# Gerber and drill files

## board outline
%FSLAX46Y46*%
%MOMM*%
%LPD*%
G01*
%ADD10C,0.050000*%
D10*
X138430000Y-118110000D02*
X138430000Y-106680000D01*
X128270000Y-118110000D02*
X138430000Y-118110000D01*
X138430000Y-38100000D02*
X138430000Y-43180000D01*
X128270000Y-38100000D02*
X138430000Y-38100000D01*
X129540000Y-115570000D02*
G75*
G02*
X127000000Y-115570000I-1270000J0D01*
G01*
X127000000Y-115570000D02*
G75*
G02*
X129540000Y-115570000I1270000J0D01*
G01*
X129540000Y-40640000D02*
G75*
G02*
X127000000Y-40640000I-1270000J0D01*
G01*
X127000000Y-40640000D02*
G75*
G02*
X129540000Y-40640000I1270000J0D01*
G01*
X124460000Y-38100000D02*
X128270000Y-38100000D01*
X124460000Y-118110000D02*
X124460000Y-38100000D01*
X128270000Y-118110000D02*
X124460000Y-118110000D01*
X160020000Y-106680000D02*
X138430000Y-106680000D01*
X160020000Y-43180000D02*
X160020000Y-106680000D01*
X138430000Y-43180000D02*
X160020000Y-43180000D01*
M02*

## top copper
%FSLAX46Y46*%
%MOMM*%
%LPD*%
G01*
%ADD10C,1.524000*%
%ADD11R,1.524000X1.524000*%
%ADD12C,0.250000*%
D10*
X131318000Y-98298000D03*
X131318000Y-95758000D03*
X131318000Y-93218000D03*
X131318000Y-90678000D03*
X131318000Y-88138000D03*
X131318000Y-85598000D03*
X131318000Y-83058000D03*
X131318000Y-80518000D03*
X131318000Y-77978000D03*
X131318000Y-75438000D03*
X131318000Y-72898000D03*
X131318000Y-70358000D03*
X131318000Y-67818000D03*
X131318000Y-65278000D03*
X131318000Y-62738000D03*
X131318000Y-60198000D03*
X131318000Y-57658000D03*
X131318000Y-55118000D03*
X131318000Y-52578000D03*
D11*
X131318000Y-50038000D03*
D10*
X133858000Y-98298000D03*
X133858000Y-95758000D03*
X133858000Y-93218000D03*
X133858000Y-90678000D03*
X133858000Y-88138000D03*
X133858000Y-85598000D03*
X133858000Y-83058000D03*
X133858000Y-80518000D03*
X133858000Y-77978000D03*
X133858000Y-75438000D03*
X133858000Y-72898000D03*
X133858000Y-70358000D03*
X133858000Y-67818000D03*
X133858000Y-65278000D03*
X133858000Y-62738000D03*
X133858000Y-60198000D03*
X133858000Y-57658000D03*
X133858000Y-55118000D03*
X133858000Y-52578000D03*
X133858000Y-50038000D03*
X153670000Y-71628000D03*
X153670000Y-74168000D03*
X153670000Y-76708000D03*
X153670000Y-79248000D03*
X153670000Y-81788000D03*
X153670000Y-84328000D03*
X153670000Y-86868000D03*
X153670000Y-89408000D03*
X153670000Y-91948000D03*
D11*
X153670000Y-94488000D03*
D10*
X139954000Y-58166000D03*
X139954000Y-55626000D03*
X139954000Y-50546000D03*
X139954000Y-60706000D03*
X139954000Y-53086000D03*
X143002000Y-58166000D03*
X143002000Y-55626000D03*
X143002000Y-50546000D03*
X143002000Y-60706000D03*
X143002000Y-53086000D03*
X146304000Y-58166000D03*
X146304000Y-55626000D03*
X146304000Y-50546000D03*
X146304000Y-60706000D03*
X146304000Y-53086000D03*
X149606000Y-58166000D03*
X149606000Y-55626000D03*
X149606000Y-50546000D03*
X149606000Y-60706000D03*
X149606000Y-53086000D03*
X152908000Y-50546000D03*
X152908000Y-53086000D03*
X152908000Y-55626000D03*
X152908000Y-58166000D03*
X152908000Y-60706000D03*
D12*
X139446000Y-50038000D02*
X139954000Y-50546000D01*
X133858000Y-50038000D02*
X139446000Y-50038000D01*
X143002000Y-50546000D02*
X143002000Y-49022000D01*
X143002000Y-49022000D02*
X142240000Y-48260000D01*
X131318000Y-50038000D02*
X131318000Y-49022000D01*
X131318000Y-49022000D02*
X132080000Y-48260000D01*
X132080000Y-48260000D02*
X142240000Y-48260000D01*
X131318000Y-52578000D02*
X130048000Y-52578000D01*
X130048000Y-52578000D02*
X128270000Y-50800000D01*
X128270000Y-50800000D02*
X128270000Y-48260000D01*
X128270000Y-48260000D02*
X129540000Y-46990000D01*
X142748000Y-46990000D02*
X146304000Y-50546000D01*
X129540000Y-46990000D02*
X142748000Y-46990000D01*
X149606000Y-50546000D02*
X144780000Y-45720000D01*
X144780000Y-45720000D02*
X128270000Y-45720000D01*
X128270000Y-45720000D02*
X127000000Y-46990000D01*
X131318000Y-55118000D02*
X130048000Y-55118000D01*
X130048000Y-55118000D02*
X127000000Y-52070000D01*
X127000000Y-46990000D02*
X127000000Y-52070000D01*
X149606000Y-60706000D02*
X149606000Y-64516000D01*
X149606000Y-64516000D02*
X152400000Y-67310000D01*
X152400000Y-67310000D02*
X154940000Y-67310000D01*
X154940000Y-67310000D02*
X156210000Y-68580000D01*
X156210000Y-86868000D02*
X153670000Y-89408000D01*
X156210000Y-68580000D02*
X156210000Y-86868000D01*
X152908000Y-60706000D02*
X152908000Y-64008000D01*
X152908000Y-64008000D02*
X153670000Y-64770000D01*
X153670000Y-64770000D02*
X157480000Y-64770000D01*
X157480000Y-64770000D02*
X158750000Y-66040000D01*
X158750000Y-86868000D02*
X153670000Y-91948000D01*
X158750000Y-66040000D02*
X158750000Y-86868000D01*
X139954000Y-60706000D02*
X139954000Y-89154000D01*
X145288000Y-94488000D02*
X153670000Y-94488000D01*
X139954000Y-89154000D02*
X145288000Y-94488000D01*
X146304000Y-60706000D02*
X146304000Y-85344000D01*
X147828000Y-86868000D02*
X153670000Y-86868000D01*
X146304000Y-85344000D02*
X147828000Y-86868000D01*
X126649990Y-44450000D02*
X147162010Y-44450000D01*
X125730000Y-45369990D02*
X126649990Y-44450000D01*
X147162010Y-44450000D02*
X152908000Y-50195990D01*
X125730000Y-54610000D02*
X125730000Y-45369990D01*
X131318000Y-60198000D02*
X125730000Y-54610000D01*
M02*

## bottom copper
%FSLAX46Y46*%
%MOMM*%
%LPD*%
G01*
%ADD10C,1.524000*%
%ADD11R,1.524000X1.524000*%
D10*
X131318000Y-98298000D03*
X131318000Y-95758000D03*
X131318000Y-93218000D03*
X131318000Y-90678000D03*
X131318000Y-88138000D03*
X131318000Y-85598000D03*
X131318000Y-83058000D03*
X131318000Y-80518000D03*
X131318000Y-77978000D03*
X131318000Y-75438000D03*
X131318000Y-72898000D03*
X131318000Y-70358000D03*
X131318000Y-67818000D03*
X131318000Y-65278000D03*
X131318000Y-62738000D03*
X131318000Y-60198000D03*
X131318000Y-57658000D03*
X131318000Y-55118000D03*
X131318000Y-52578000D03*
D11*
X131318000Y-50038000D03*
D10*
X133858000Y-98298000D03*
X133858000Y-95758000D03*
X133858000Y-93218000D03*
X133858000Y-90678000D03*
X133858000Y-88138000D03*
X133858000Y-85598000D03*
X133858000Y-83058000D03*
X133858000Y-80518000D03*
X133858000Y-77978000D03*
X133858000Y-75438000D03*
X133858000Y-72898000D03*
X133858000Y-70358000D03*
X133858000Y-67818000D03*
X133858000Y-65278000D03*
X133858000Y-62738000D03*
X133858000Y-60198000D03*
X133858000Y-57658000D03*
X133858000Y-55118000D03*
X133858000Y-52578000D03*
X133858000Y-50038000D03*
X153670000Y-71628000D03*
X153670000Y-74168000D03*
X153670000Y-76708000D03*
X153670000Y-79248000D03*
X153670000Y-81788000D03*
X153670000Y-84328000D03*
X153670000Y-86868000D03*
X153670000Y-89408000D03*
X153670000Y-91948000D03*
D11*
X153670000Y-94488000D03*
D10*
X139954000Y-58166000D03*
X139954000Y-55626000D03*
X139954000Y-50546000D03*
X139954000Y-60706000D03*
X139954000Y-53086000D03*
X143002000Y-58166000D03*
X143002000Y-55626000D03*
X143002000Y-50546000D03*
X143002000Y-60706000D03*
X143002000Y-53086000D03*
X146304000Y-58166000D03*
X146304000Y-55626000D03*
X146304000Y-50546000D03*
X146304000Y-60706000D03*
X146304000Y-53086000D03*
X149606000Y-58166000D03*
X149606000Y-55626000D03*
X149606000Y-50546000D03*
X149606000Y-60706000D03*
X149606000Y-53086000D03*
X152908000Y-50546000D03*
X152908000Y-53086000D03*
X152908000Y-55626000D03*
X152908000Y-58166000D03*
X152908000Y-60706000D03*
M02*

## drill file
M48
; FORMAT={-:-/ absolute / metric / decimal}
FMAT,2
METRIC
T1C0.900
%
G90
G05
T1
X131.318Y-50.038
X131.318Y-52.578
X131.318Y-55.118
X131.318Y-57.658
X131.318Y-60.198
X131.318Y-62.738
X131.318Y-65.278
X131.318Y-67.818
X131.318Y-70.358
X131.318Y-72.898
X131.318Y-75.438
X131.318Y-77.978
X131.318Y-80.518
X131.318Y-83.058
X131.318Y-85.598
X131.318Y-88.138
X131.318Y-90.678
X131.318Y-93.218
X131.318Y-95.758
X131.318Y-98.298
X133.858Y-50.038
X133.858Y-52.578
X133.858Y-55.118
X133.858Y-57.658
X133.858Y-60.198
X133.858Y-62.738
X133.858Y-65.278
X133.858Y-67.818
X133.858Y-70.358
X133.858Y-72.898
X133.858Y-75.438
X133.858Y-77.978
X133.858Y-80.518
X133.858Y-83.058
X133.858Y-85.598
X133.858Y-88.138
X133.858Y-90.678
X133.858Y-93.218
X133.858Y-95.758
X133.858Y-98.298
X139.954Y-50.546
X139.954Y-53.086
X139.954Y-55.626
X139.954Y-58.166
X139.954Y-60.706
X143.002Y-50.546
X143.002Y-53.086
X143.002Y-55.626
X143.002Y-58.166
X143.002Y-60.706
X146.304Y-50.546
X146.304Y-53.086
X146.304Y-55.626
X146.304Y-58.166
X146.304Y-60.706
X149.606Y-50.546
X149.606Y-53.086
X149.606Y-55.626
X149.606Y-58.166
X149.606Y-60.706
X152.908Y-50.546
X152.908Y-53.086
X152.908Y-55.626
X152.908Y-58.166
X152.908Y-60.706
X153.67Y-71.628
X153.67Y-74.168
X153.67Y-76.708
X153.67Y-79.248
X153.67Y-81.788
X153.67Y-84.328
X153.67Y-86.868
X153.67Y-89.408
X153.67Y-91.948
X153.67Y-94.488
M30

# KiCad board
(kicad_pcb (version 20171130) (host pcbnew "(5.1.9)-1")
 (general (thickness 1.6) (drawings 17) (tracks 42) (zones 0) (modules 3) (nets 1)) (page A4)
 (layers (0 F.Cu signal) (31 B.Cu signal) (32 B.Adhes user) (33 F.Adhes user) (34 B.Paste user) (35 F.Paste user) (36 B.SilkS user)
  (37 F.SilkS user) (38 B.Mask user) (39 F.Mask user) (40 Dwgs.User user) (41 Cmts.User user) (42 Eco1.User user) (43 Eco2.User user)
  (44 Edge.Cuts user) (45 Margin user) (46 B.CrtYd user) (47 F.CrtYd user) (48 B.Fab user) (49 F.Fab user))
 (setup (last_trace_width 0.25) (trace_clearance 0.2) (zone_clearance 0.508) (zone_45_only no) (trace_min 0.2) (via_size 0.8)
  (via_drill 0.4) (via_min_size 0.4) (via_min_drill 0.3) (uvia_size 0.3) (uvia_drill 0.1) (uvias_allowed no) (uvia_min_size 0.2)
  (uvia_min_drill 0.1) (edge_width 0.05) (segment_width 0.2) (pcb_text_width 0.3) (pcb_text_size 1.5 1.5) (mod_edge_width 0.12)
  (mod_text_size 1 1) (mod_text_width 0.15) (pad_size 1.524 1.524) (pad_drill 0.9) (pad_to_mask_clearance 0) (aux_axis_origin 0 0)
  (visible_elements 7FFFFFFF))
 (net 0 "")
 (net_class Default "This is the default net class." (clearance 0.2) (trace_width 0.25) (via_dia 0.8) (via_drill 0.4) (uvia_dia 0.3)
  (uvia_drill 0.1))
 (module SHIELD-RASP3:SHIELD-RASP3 (layer F.Cu) (at 118.11 100.33)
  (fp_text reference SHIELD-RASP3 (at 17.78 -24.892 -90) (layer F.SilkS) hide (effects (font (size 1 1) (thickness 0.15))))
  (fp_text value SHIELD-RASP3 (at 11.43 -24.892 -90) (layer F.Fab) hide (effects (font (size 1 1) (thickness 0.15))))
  (pad 39 thru_hole circle (at 13.208 -2.032 270) (size 1.524 1.524) (drill 0.9) (layers *.Cu *.Mask))
  (pad 37 thru_hole circle (at 13.208 -4.572 270) (size 1.524 1.524) (drill 0.9) (layers *.Cu *.Mask))
  (pad 35 thru_hole circle (at 13.208 -7.112 270) (size 1.524 1.524) (drill 0.9) (layers *.Cu *.Mask))
  (pad 33 thru_hole circle (at 13.208 -9.652 270) (size 1.524 1.524) (drill 0.9) (layers *.Cu *.Mask))
  (pad 31 thru_hole circle (at 13.208 -12.192 270) (size 1.524 1.524) (drill 0.9) (layers *.Cu *.Mask))
  (pad 29 thru_hole circle (at 13.208 -14.732 270) (size 1.524 1.524) (drill 0.9) (layers *.Cu *.Mask))
  (pad 27 thru_hole circle (at 13.208 -17.272 270) (size 1.524 1.524) (drill 0.9) (layers *.Cu *.Mask))
  (pad 25 thru_hole circle (at 13.208 -19.812 270) (size 1.524 1.524) (drill 0.9) (layers *.Cu *.Mask))
  (pad 23 thru_hole circle (at 13.208 -22.352 270) (size 1.524 1.524) (drill 0.9) (layers *.Cu *.Mask))
  (pad 21 thru_hole circle (at 13.208 -24.892 270) (size 1.524 1.524) (drill 0.9) (layers *.Cu *.Mask))
  (pad 19 thru_hole circle (at 13.208 -27.432 270) (size 1.524 1.524) (drill 0.9) (layers *.Cu *.Mask))
  (pad 17 thru_hole circle (at 13.208 -29.972 270) (size 1.524 1.524) (drill 0.9) (layers *.Cu *.Mask))
  (pad 15 thru_hole circle (at 13.208 -32.512 270) (size 1.524 1.524) (drill 0.9) (layers *.Cu *.Mask))
  (pad 13 thru_hole circle (at 13.208 -35.052 270) (size 1.524 1.524) (drill 0.9) (layers *.Cu *.Mask))
  (pad 11 thru_hole circle (at 13.208 -37.592 270) (size 1.524 1.524) (drill 0.9) (layers *.Cu *.Mask))
  (pad 9 thru_hole circle (at 13.208 -40.132 270) (size 1.524 1.524) (drill 0.9) (layers *.Cu *.Mask))
  (pad 7 thru_hole circle (at 13.208 -42.672 270) (size 1.524 1.524) (drill 0.9) (layers *.Cu *.Mask F.Paste))
  (pad 5 thru_hole circle (at 13.208 -45.212 270) (size 1.524 1.524) (drill 0.9) (layers *.Cu *.Mask))
  (pad 3 thru_hole circle (at 13.208 -47.752 270) (size 1.524 1.524) (drill 0.9) (layers *.Cu *.Mask))
  (pad 1 thru_hole rect (at 13.208 -50.292 270) (size 1.524 1.524) (drill 0.9) (layers *.Cu *.Mask))
  (pad 40 thru_hole circle (at 15.748 -2.032 270) (size 1.524 1.524) (drill 0.9) (layers *.Cu *.Mask))
  (pad 38 thru_hole circle (at 15.748 -4.572 270) (size 1.524 1.524) (drill 0.9) (layers *.Cu *.Mask))
  (pad 36 thru_hole circle (at 15.748 -7.112 270) (size 1.524 1.524) (drill 0.9) (layers *.Cu *.Mask))
  (pad 34 thru_hole circle (at 15.748 -9.652 270) (size 1.524 1.524) (drill 0.9) (layers *.Cu *.Mask))
  (pad 32 thru_hole circle (at 15.748 -12.192 270) (size 1.524 1.524) (drill 0.9) (layers *.Cu *.Mask))
  (pad 30 thru_hole circle (at 15.748 -14.732 270) (size 1.524 1.524) (drill 0.9) (layers *.Cu *.Mask))
  (pad 28 thru_hole circle (at 15.748 -17.272 270) (size 1.524 1.524) (drill 0.9) (layers *.Cu *.Mask))
  (pad 26 thru_hole circle (at 15.748 -19.812 270) (size 1.524 1.524) (drill 0.9) (layers *.Cu *.Mask))
  (pad 24 thru_hole circle (at 15.748 -22.352 270) (size 1.524 1.524) (drill 0.9) (layers *.Cu *.Mask))
  (pad 22 thru_hole circle (at 15.748 -24.892 270) (size 1.524 1.524) (drill 0.9) (layers *.Cu *.Mask))
  (pad 20 thru_hole circle (at 15.748 -27.432 270) (size 1.524 1.524) (drill 0.9) (layers *.Cu *.Mask))
  (pad 18 thru_hole circle (at 15.748 -29.972 270) (size 1.524 1.524) (drill 0.9) (layers *.Cu *.Mask))
  (pad 16 thru_hole circle (at 15.748 -32.512 270) (size 1.524 1.524) (drill 0.9) (layers *.Cu *.Mask))
  (pad 14 thru_hole circle (at 15.748 -35.052 270) (size 1.524 1.524) (drill 0.9) (layers *.Cu *.Mask))
  (pad 12 thru_hole circle (at 15.748 -37.592 270) (size 1.524 1.524) (drill 0.9) (layers *.Cu *.Mask))
  (pad 10 thru_hole circle (at 15.748 -40.132 270) (size 1.524 1.524) (drill 0.9) (layers *.Cu *.Mask))
  (pad 8 thru_hole circle (at 15.748 -42.672 270) (size 1.524 1.524) (drill 0.9) (layers *.Cu *.Mask))
  (pad 6 thru_hole circle (at 15.748 -45.212 270) (size 1.524 1.524) (drill 0.9) (layers *.Cu *.Mask))
  (pad 4 thru_hole circle (at 15.748 -47.752 270) (size 1.524 1.524) (drill 0.9) (layers *.Cu *.Mask))
  (pad 2 thru_hole circle (at 15.748 -50.292 270) (size 1.524 1.524) (drill 0.9) (layers *.Cu *.Mask)))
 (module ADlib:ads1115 (layer F.Cu) (at 148.59 92.71 90)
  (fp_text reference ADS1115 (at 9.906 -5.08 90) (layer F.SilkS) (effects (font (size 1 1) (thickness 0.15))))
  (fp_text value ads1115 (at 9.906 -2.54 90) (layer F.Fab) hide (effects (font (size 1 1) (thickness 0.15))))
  (pad 10 thru_hole circle (at 21.082 5.08 90) (size 1.524 1.524) (drill 0.9) (layers *.Cu *.Mask))
  (pad 9 thru_hole circle (at 18.542 5.08 90) (size 1.524 1.524) (drill 0.9) (layers *.Cu *.Mask))
  (pad 8 thru_hole circle (at 16.002 5.08 90) (size 1.524 1.524) (drill 0.9) (layers *.Cu *.Mask))
  (pad 7 thru_hole circle (at 13.462 5.08 90) (size 1.524 1.524) (drill 0.9) (layers *.Cu *.Mask))
  (pad 6 thru_hole circle (at 10.922 5.08 90) (size 1.524 1.524) (drill 0.9) (layers *.Cu *.Mask))
  (pad 5 thru_hole circle (at 8.382 5.08 90) (size 1.524 1.524) (drill 0.9) (layers *.Cu *.Mask))
  (pad 4 thru_hole circle (at 5.842 5.08 90) (size 1.524 1.524) (drill 0.9) (layers *.Cu *.Mask))
  (pad 3 thru_hole circle (at 3.302 5.08 90) (size 1.524 1.524) (drill 0.9) (layers *.Cu *.Mask))
  (pad 2 thru_hole circle (at 0.762 5.08 90) (size 1.524 1.524) (drill 0.9) (layers *.Cu *.Mask))
  (pad 1 thru_hole rect (at -1.778 5.08 90) (size 1.524 1.524) (drill 0.9) (layers *.Cu *.Mask)))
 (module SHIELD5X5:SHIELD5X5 (layer F.Cu) (at 154.94 54.61 180)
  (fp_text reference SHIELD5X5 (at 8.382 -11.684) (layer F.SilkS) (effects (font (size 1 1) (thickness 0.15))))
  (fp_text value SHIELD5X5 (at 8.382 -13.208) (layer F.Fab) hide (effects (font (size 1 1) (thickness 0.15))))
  (pad 2 thru_hole circle (at 14.986 -3.556 180) (size 1.524 1.524) (drill 0.9) (layers *.Cu *.Mask))
  (pad 3 thru_hole circle (at 14.986 -1.016 180) (size 1.524 1.524) (drill 0.9) (layers *.Cu *.Mask))
  (pad 5 thru_hole circle (at 14.986 4.064 180) (size 1.524 1.524) (drill 0.9) (layers *.Cu *.Mask))
  (pad 1 thru_hole circle (at 14.986 -6.096 180) (size 1.524 1.524) (drill 0.9) (layers *.Cu *.Mask))
  (pad 4 thru_hole circle (at 14.986 1.524 180) (size 1.524 1.524) (drill 0.9) (layers *.Cu *.Mask))
  (pad 2 thru_hole circle (at 11.938 -3.556 180) (size 1.524 1.524) (drill 0.9) (layers *.Cu *.Mask))
  (pad 3 thru_hole circle (at 11.938 -1.016 180) (size 1.524 1.524) (drill 0.9) (layers *.Cu *.Mask))
  (pad 5 thru_hole circle (at 11.938 4.064 180) (size 1.524 1.524) (drill 0.9) (layers *.Cu *.Mask))
  (pad 1 thru_hole circle (at 11.938 -6.096 180) (size 1.524 1.524) (drill 0.9) (layers *.Cu *.Mask))
  (pad 4 thru_hole circle (at 11.938 1.524 180) (size 1.524 1.524) (drill 0.9) (layers *.Cu *.Mask))
  (pad 2 thru_hole circle (at 8.636 -3.556 180) (size 1.524 1.524) (drill 0.9) (layers *.Cu *.Mask))
  (pad 3 thru_hole circle (at 8.636 -1.016 180) (size 1.524 1.524) (drill 0.9) (layers *.Cu *.Mask))
  (pad 5 thru_hole circle (at 8.636 4.064 180) (size 1.524 1.524) (drill 0.9) (layers *.Cu *.Mask))
  (pad 1 thru_hole circle (at 8.636 -6.096 180) (size 1.524 1.524) (drill 0.9) (layers *.Cu *.Mask))
  (pad 4 thru_hole circle (at 8.636 1.524 180) (size 1.524 1.524) (drill 0.9) (layers *.Cu *.Mask))
  (pad 2 thru_hole circle (at 5.334 -3.556 180) (size 1.524 1.524) (drill 0.9) (layers *.Cu *.Mask))
  (pad 3 thru_hole circle (at 5.334 -1.016 180) (size 1.524 1.524) (drill 0.9) (layers *.Cu *.Mask))
  (pad 5 thru_hole circle (at 5.334 4.064 180) (size 1.524 1.524) (drill 0.9) (layers *.Cu *.Mask))
  (pad 1 thru_hole circle (at 5.334 -6.096 180) (size 1.524 1.524) (drill 0.9) (layers *.Cu *.Mask))
  (pad 4 thru_hole circle (at 5.334 1.524 180) (size 1.524 1.524) (drill 0.9) (layers *.Cu *.Mask))
  (pad 5 thru_hole circle (at 2.032 4.064 180) (size 1.524 1.524) (drill 0.9) (layers *.Cu *.Mask))
  (pad 4 thru_hole circle (at 2.032 1.524 180) (size 1.524 1.524) (drill 0.9) (layers *.Cu *.Mask))
  (pad 3 thru_hole circle (at 2.032 -1.016 180) (size 1.524 1.524) (drill 0.9) (layers *.Cu *.Mask))
  (pad 2 thru_hole circle (at 2.032 -3.556 180) (size 1.524 1.524) (drill 0.9) (layers *.Cu *.Mask))
  (pad 1 thru_hole circle (at 2.032 -6.096 180) (size 1.524 1.524) (drill 0.9) (layers *.Cu *.Mask)))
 (gr_line (start 138.43 118.11) (end 138.43 106.68) (layer Edge.Cuts) (width 0.05))
 (gr_line (start 128.27 118.11) (end 138.43 118.11) (layer Edge.Cuts) (width 0.05))
 (gr_line (start 138.43 38.1) (end 138.43 43.18) (layer Edge.Cuts) (width 0.05))
 (gr_line (start 128.27 38.1) (end 138.43 38.1) (layer Edge.Cuts) (width 0.05))
 (gr_circle (center 128.27 115.57) (end 129.54 115.57) (layer Edge.Cuts) (width 0.05))
 (gr_circle (center 128.27 40.64) (end 129.54 40.64) (layer Edge.Cuts) (width 0.05))
 (gr_line (start 124.46 38.1) (end 128.27 38.1) (layer Edge.Cuts) (width 0.05))
 (gr_line (start 124.46 118.11) (end 124.46 38.1) (layer Edge.Cuts) (width 0.05))
 (gr_line (start 128.27 118.11) (end 124.46 118.11) (layer Edge.Cuts) (width 0.05))
 (gr_line (start 160.02 106.68) (end 138.43 106.68) (layer Edge.Cuts) (width 0.05))
 (gr_line (start 160.02 43.18) (end 160.02 106.68) (layer Edge.Cuts) (width 0.05))
 (gr_line (start 138.43 43.18) (end 160.02 43.18) (layer Edge.Cuts) (width 0.05))
 (segment (start 139.446 50.038) (end 139.954 50.546) (width 0.25) (layer F.Cu) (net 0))
 (segment (start 133.858 50.038) (end 139.446 50.038) (width 0.25) (layer F.Cu) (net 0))
 (segment (start 143.002 50.546) (end 143.002 49.022) (width 0.25) (layer F.Cu) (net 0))
 (segment (start 143.002 49.022) (end 142.24 48.26) (width 0.25) (layer F.Cu) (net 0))
 (segment (start 131.318 50.038) (end 131.318 49.022) (width 0.25) (layer F.Cu) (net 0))
 (segment (start 131.318 49.022) (end 132.08 48.26) (width 0.25) (layer F.Cu) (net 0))
 (segment (start 132.08 48.26) (end 142.24 48.26) (width 0.25) (layer F.Cu) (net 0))
 (segment (start 131.318 52.578) (end 130.048 52.578) (width 0.25) (layer F.Cu) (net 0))
 (segment (start 130.048 52.578) (end 128.27 50.8) (width 0.25) (layer F.Cu) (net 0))
 (segment (start 128.27 50.8) (end 128.27 48.26) (width 0.25) (layer F.Cu) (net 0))
 (segment (start 128.27 48.26) (end 129.54 46.99) (width 0.25) (layer F.Cu) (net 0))
 (segment (start 142.748 46.99) (end 146.304 50.546) (width 0.25) (layer F.Cu) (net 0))
 (segment (start 129.54 46.99) (end 142.748 46.99) (width 0.25) (layer F.Cu) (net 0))
 (segment (start 149.606 50.546) (end 144.78 45.72) (width 0.25) (layer F.Cu) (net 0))
 (segment (start 144.78 45.72) (end 128.27 45.72) (width 0.25) (layer F.Cu) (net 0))
 (segment (start 128.27 45.72) (end 127 46.99) (width 0.25) (layer F.Cu) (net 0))
 (segment (start 131.318 55.118) (end 130.048 55.118) (width 0.25) (layer F.Cu) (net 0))
 (segment (start 130.048 55.118) (end 127 52.07) (width 0.25) (layer F.Cu) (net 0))
 (segment (start 127 46.99) (end 127 52.07) (width 0.25) (layer F.Cu) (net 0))
 (segment (start 149.606 60.706) (end 149.606 64.516) (width 0.25) (layer F.Cu) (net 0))
 (segment (start 149.606 64.516) (end 152.4 67.31) (width 0.25) (layer F.Cu) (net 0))
 (segment (start 152.4 67.31) (end 154.94 67.31) (width 0.25) (layer F.Cu) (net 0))
 (segment (start 154.94 67.31) (end 156.21 68.58) (width 0.25) (layer F.Cu) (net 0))
 (segment (start 156.21 86.868) (end 153.67 89.408) (width 0.25) (layer F.Cu) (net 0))
 (segment (start 156.21 68.58) (end 156.21 86.868) (width 0.25) (layer F.Cu) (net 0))
 (segment (start 152.908 60.706) (end 152.908 64.008) (width 0.25) (layer F.Cu) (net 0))
 (segment (start 152.908 64.008) (end 153.67 64.77) (width 0.25) (layer F.Cu) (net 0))
 (segment (start 153.67 64.77) (end 157.48 64.77) (width 0.25) (layer F.Cu) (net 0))
 (segment (start 157.48 64.77) (end 158.75 66.04) (width 0.25) (layer F.Cu) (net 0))
 (segment (start 158.75 86.868) (end 153.67 91.948) (width 0.25) (layer F.Cu) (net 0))
 (segment (start 158.75 66.04) (end 158.75 86.868) (width 0.25) (layer F.Cu) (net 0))
 (segment (start 139.954 60.706) (end 139.954 89.154) (width 0.25) (layer F.Cu) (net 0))
 (segment (start 145.288 94.488) (end 153.67 94.488) (width 0.25) (layer F.Cu) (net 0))
 (segment (start 139.954 89.154) (end 145.288 94.488) (width 0.25) (layer F.Cu) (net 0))
 (segment (start 146.304 60.706) (end 146.304 85.344) (width 0.25) (layer F.Cu) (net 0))
 (segment (start 147.828 86.868) (end 153.67 86.868) (width 0.25) (layer F.Cu) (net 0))
 (segment (start 146.304 85.344) (end 147.828 86.868) (width 0.25) (layer F.Cu) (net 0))
 (segment (start 126.64999 44.45) (end 147.16201 44.45) (width 0.25) (layer F.Cu) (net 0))
 (segment (start 125.73 45.36999) (end 126.64999 44.45) (width 0.25) (layer F.Cu) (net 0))
 (segment (start 147.16201 44.45) (end 152.908 50.19599) (width 0.25) (layer F.Cu) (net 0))
 (segment (start 125.73 54.61) (end 125.73 45.36999) (width 0.25) (layer F.Cu) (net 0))
 (segment (start 131.318 60.198) (end 125.73 54.61) (width 0.25) (layer F.Cu) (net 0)))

